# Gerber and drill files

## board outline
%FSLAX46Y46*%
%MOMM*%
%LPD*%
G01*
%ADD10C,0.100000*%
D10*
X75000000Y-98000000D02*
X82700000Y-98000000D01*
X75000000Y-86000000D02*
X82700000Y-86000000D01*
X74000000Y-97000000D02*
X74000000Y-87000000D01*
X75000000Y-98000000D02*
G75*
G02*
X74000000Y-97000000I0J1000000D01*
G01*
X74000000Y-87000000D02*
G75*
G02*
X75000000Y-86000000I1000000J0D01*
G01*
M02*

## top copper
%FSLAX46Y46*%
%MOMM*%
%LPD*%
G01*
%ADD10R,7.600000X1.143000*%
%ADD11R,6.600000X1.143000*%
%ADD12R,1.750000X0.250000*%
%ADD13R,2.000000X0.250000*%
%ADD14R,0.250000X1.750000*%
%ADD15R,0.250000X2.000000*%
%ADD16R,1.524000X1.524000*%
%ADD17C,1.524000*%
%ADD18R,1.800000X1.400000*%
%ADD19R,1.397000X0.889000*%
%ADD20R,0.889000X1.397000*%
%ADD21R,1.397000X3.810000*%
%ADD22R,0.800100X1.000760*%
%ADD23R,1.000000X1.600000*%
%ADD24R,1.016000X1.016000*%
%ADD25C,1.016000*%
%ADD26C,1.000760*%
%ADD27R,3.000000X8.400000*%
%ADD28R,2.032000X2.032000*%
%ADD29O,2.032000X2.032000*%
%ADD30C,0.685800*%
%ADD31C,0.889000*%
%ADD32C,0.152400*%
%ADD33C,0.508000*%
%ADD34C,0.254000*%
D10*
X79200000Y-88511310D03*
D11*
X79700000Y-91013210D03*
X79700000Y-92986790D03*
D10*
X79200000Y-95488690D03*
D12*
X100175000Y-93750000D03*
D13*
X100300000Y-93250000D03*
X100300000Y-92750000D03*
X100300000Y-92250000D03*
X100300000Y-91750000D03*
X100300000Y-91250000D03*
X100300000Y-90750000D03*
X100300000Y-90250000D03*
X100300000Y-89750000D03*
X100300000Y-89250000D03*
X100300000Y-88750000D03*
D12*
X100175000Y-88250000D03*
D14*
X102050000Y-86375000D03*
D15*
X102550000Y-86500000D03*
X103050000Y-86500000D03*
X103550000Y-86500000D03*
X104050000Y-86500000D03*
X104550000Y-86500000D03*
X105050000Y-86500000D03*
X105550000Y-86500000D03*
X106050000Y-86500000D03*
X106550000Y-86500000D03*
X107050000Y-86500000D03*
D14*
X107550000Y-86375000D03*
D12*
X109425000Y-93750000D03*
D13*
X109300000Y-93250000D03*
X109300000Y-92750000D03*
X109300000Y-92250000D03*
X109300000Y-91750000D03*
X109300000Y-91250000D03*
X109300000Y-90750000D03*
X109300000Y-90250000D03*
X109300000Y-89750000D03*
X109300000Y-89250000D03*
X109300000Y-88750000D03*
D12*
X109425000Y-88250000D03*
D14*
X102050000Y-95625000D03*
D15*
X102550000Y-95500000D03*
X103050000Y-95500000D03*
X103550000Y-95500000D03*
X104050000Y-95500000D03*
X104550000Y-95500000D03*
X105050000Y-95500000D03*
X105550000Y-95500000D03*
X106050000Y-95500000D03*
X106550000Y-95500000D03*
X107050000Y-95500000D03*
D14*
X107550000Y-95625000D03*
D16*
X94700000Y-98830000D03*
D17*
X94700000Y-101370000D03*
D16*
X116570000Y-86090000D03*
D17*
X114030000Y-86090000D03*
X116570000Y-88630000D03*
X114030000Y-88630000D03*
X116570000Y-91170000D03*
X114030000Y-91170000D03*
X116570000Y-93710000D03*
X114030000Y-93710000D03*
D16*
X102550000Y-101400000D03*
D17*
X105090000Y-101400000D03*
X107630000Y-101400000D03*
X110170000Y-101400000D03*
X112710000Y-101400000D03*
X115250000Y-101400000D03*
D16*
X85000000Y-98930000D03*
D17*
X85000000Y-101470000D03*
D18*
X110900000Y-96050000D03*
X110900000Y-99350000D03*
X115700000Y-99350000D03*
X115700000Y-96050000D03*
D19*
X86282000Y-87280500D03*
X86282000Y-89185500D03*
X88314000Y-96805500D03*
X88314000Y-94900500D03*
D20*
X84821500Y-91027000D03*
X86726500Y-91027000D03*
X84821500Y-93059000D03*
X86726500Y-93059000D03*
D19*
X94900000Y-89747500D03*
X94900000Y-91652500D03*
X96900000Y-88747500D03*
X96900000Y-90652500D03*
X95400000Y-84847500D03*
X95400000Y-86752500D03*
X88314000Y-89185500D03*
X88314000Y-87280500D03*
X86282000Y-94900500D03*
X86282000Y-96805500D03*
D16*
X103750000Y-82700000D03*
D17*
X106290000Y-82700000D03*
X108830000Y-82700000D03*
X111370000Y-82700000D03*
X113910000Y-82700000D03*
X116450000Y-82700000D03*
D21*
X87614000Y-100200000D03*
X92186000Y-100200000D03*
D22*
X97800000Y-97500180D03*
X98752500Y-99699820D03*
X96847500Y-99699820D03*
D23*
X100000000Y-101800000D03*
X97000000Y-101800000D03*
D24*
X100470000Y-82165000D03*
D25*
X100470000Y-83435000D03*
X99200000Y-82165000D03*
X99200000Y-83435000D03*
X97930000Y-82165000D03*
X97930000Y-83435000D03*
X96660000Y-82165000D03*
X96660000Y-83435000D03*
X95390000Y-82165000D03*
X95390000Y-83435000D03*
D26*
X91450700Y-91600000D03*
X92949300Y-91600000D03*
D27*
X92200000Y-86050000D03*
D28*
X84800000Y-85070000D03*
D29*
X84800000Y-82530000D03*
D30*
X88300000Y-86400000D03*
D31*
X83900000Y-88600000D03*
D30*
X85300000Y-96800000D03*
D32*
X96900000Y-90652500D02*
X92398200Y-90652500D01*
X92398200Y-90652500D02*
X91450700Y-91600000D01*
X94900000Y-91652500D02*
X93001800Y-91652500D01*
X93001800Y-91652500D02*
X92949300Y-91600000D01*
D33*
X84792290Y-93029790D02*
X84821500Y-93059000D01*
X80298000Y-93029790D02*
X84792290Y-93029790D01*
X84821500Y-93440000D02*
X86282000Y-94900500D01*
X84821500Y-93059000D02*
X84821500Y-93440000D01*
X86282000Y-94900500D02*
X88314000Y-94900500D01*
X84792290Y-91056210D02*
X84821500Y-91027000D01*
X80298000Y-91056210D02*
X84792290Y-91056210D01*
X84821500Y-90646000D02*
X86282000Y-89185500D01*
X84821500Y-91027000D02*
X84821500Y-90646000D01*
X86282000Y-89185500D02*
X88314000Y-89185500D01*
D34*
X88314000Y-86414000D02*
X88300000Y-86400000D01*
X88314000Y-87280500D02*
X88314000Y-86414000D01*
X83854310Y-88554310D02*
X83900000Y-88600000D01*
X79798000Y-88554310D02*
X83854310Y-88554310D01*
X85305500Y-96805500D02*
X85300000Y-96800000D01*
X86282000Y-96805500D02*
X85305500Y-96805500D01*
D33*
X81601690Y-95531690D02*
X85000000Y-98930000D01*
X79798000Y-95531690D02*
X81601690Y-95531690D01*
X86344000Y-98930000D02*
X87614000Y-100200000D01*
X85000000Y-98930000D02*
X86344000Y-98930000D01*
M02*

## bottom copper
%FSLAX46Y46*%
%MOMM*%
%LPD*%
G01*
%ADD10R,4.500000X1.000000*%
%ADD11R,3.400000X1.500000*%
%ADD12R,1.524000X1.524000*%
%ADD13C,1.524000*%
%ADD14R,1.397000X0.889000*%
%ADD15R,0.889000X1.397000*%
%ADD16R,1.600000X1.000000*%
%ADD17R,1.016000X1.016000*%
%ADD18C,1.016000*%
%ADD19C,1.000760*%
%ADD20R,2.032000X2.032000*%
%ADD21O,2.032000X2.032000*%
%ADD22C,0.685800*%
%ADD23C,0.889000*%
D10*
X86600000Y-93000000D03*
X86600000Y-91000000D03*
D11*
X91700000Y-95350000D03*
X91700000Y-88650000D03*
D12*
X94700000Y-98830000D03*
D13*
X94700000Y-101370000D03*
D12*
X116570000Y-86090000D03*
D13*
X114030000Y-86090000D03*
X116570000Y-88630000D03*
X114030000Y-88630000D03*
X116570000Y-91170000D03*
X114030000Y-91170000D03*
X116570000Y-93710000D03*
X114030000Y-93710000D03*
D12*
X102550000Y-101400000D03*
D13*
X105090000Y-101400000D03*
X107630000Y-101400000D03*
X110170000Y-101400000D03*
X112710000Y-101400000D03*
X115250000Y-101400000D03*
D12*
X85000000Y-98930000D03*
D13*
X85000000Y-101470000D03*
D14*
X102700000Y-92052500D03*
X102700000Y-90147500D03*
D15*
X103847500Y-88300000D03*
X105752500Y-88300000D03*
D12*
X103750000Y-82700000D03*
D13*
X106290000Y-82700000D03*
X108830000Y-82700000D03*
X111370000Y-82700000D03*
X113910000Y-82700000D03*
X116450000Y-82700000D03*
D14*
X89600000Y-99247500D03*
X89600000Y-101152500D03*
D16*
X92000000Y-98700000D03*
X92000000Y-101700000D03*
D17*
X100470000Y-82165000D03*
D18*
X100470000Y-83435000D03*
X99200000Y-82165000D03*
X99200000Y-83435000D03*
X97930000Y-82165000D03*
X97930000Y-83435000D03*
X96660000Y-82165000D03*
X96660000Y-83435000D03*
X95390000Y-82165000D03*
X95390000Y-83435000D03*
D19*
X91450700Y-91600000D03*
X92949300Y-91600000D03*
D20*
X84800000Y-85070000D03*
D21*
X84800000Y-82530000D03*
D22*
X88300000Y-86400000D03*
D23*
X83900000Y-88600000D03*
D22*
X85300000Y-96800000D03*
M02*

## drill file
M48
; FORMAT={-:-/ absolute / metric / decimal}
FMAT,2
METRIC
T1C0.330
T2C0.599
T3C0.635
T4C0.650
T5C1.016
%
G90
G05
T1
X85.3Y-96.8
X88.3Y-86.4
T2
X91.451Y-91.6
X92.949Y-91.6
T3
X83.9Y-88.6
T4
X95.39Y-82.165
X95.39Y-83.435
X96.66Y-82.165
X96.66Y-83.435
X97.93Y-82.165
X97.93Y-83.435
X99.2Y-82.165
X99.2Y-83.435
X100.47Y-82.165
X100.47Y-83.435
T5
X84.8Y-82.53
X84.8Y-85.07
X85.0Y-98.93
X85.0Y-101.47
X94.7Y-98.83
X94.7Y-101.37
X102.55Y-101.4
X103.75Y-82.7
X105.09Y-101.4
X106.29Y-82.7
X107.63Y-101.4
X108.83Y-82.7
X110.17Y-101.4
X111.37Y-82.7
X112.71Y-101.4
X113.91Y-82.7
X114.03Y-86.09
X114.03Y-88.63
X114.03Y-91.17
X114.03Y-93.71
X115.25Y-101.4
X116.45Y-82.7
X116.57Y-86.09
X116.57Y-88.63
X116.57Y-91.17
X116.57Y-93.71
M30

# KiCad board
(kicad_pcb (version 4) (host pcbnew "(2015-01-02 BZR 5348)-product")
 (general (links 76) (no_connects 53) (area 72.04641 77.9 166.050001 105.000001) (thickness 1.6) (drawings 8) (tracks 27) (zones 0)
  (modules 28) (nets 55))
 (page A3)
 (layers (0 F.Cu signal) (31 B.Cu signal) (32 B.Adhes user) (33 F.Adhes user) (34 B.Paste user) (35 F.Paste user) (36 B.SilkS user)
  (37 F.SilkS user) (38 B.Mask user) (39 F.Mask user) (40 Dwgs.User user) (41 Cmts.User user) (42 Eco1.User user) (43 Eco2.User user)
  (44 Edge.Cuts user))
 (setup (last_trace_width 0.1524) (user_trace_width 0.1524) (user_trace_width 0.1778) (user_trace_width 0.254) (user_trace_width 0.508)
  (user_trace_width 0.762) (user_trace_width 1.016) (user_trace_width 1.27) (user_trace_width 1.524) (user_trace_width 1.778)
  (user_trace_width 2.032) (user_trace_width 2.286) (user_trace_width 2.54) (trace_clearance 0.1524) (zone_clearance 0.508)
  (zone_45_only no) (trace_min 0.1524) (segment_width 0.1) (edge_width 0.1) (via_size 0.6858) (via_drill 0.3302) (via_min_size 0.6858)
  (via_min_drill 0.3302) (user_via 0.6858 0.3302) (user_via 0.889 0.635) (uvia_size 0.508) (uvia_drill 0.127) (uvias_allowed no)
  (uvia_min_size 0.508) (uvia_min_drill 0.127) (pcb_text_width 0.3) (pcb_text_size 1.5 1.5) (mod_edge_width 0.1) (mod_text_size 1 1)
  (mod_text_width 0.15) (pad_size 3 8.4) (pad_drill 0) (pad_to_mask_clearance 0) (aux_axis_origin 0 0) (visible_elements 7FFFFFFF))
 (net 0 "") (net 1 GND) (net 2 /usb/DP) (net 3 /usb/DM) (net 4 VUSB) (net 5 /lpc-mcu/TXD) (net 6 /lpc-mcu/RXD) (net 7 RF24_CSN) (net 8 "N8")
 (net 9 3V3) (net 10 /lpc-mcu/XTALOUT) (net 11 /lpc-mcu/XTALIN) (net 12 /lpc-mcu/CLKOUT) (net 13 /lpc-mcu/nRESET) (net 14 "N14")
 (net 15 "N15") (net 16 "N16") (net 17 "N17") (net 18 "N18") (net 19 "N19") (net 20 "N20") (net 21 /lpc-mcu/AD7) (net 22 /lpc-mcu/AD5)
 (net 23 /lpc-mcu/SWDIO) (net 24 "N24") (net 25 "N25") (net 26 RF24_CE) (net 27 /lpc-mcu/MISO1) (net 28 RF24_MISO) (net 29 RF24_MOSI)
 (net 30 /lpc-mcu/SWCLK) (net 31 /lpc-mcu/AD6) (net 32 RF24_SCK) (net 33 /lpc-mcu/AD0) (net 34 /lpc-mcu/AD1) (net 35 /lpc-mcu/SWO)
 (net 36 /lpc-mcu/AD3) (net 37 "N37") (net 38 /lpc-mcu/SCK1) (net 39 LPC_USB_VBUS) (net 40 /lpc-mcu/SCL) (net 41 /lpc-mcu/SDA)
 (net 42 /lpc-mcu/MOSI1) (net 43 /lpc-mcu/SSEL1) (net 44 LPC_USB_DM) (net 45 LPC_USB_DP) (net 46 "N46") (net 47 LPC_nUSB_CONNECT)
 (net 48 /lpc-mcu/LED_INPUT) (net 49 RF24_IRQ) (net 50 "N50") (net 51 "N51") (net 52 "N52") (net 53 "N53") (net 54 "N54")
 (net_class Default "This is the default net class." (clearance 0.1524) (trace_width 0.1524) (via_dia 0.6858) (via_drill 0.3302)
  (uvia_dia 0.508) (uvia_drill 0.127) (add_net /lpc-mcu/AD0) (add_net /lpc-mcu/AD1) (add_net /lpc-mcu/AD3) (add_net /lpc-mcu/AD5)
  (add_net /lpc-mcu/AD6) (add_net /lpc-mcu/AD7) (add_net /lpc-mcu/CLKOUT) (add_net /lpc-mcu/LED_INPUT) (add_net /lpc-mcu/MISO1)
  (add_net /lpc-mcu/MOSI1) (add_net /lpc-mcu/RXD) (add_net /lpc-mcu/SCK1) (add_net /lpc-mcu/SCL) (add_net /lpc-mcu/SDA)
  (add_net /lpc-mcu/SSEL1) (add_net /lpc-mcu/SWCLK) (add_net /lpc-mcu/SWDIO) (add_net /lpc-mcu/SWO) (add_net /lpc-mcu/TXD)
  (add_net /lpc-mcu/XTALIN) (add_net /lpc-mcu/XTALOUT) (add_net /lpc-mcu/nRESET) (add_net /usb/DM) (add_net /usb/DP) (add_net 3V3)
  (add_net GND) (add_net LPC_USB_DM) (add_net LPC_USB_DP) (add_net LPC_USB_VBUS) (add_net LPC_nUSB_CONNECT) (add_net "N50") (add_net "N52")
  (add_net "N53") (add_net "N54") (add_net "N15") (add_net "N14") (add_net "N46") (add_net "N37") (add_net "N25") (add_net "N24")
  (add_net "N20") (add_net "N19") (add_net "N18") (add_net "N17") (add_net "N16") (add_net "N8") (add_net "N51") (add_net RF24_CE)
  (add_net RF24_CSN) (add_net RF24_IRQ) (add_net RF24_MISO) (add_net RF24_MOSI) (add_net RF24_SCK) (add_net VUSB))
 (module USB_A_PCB (layer F.Cu) (at 74 92 270)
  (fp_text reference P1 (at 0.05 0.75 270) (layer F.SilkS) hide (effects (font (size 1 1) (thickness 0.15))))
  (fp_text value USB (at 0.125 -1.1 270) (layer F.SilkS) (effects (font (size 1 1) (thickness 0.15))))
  (pad 4 smd rect (at -3.48869 -5.2 270) (size 1.143 7.6) (layers F.Cu F.Paste F.Mask) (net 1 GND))
  (pad 3 smd rect (at -0.98679 -5.7 270) (size 1.143 6.6) (layers F.Cu F.Paste F.Mask) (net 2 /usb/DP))
  (pad 2 smd rect (at 0.98679 -5.7 270) (size 1.143 6.6) (layers F.Cu F.Paste F.Mask) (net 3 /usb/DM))
  (pad 1 smd rect (at 3.48869 -5.2 270) (size 1.143 7.6) (layers F.Cu F.Paste F.Mask) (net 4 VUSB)))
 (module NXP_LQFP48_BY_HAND (layer F.Cu) (at 104.8 91) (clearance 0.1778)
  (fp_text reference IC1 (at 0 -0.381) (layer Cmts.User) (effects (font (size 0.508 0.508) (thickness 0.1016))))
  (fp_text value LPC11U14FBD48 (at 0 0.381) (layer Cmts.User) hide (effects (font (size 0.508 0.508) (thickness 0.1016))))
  (pad 12 smd rect (at -4.625 2.75) (size 1.75 0.25) (layers F.Cu F.Paste F.Mask) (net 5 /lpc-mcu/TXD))
  (pad 11 smd rect (at -4.5 2.25) (size 2 0.25) (layers F.Cu F.Paste F.Mask) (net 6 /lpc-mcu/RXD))
  (pad 10 smd rect (at -4.5 1.75) (size 2 0.25) (layers F.Cu F.Paste F.Mask) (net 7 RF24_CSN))
  (pad 9 smd rect (at -4.5 1.25) (size 2 0.25) (layers F.Cu F.Paste F.Mask) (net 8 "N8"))
  (pad 8 smd rect (at -4.5 0.75) (size 2 0.25) (layers F.Cu F.Paste F.Mask) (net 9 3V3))
  (pad 7 smd rect (at -4.5 0.25) (size 2 0.25) (layers F.Cu F.Paste F.Mask) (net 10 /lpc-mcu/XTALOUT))
  (pad 6 smd rect (at -4.5 -0.25) (size 2 0.25) (layers F.Cu F.Paste F.Mask) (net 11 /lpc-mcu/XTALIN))
  (pad 5 smd rect (at -4.5 -0.75) (size 2 0.25) (layers F.Cu F.Paste F.Mask) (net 1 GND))
  (pad 4 smd rect (at -4.5 -1.25) (size 2 0.25) (layers F.Cu F.Paste F.Mask) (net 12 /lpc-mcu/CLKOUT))
  (pad 3 smd rect (at -4.5 -1.75) (size 2 0.25) (layers F.Cu F.Paste F.Mask) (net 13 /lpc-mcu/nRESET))
  (pad 2 smd rect (at -4.5 -2.25) (size 2 0.25) (layers F.Cu F.Paste F.Mask) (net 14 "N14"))
  (pad 1 smd rect (at -4.625 -2.75) (size 1.75 0.25) (layers F.Cu F.Paste F.Mask) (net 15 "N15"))
  (pad 48 smd rect (at -2.75 -4.625) (size 0.25 1.75) (layers F.Cu F.Paste F.Mask) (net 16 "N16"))
  (pad 47 smd rect (at -2.25 -4.5) (size 0.25 2) (layers F.Cu F.Paste F.Mask) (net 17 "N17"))
  (pad 46 smd rect (at -1.75 -4.5) (size 0.25 2) (layers F.Cu F.Paste F.Mask) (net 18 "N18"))
  (pad 45 smd rect (at -1.25 -4.5) (size 0.25 2) (layers F.Cu F.Paste F.Mask) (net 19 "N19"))
  (pad 44 smd rect (at -0.75 -4.5) (size 0.25 2) (layers F.Cu F.Paste F.Mask) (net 9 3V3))
  (pad 43 smd rect (at -0.25 -4.5) (size 0.25 2) (layers F.Cu F.Paste F.Mask) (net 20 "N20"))
  (pad 42 smd rect (at 0.25 -4.5) (size 0.25 2) (layers F.Cu F.Paste F.Mask) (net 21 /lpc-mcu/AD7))
  (pad 41 smd rect (at 0.75 -4.5) (size 0.25 2) (layers F.Cu F.Paste F.Mask) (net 1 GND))
  (pad 40 smd rect (at 1.25 -4.5) (size 0.25 2) (layers F.Cu F.Paste F.Mask) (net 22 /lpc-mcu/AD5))
  (pad 39 smd rect (at 1.75 -4.5) (size 0.25 2) (layers F.Cu F.Paste F.Mask) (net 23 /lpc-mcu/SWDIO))
  (pad 38 smd rect (at 2.25 -4.5) (size 0.25 2) (layers F.Cu F.Paste F.Mask) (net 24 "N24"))
  (pad 37 smd rect (at 2.75 -4.625) (size 0.25 1.75) (layers F.Cu F.Paste F.Mask) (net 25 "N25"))
  (pad 25 smd rect (at 4.625 2.75) (size 1.75 0.25) (layers F.Cu F.Paste F.Mask) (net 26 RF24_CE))
  (pad 26 smd rect (at 4.5 2.25) (size 2 0.25) (layers F.Cu F.Paste F.Mask) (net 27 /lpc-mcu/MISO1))
  (pad 27 smd rect (at 4.5 1.75) (size 2 0.25) (layers F.Cu F.Paste F.Mask) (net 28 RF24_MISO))
  (pad 28 smd rect (at 4.5 1.25) (size 2 0.25) (layers F.Cu F.Paste F.Mask) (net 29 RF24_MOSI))
  (pad 29 smd rect (at 4.5 0.75) (size 2 0.25) (layers F.Cu F.Paste F.Mask) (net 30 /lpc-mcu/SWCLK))
  (pad 30 smd rect (at 4.5 0.25) (size 2 0.25) (layers F.Cu F.Paste F.Mask) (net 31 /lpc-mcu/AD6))
  (pad 31 smd rect (at 4.5 -0.25) (size 2 0.25) (layers F.Cu F.Paste F.Mask) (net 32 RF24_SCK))
  (pad 32 smd rect (at 4.5 -0.75) (size 2 0.25) (layers F.Cu F.Paste F.Mask) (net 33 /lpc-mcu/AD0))
  (pad 33 smd rect (at 4.5 -1.25) (size 2 0.25) (layers F.Cu F.Paste F.Mask) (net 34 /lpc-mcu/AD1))
  (pad 34 smd rect (at 4.5 -1.75) (size 2 0.25) (layers F.Cu F.Paste F.Mask) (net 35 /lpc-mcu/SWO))
  (pad 35 smd rect (at 4.5 -2.25) (size 2 0.25) (layers F.Cu F.Paste F.Mask) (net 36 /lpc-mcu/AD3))
  (pad 36 smd rect (at 4.625 -2.75) (size 1.75 0.25) (layers F.Cu F.Paste F.Mask) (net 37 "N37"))
  (pad 13 smd rect (at -2.75 4.625) (size 0.25 1.75) (layers F.Cu F.Paste F.Mask) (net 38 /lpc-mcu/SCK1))
  (pad 14 smd rect (at -2.25 4.5) (size 0.25 2) (layers F.Cu F.Paste F.Mask) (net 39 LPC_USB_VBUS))
  (pad 15 smd rect (at -1.75 4.5) (size 0.25 2) (layers F.Cu F.Paste F.Mask) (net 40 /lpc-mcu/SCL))
  (pad 16 smd rect (at -1.25 4.5) (size 0.25 2) (layers F.Cu F.Paste F.Mask) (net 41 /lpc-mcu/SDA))
  (pad 17 smd rect (at -0.75 4.5) (size 0.25 2) (layers F.Cu F.Paste F.Mask) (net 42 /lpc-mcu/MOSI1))
  (pad 18 smd rect (at -0.25 4.5) (size 0.25 2) (layers F.Cu F.Paste F.Mask) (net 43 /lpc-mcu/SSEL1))
  (pad 19 smd rect (at 0.25 4.5) (size 0.25 2) (layers F.Cu F.Paste F.Mask) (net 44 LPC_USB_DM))
  (pad 20 smd rect (at 0.75 4.5) (size 0.25 2) (layers F.Cu F.Paste F.Mask) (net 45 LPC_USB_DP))
  (pad 21 smd rect (at 1.25 4.5) (size 0.25 2) (layers F.Cu F.Paste F.Mask) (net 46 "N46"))
  (pad 22 smd rect (at 1.75 4.5) (size 0.25 2) (layers F.Cu F.Paste F.Mask) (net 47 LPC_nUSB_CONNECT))
  (pad 23 smd rect (at 2.25 4.5) (size 0.25 2) (layers F.Cu F.Paste F.Mask) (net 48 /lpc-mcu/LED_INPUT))
  (pad 24 smd rect (at 2.75 4.625) (size 0.25 1.75) (layers F.Cu F.Paste F.Mask) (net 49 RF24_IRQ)))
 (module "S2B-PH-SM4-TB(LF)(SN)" (layer B.Cu) (at 86.6 92 90)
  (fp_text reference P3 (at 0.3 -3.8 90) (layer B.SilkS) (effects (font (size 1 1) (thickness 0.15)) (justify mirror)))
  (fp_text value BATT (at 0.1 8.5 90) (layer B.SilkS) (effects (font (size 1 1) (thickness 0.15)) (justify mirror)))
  (pad 1 smd rect (at -1 0 90) (size 1 4.5) (layers B.Cu B.Paste B.Mask) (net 1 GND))
  (pad 2 smd rect (at 1 0 90) (size 1 4.5) (layers B.Cu B.Paste B.Mask) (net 4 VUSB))
  (pad NC smd rect (at -3.35 5.1 90) (size 1.5 3.4) (layers B.Cu B.Paste B.Mask))
  (pad NC smd rect (at 3.35 5.1 90) (size 1.5 3.4) (layers B.Cu B.Paste B.Mask)))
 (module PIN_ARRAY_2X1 (layer F.Cu) (at 94.7 100.1 270)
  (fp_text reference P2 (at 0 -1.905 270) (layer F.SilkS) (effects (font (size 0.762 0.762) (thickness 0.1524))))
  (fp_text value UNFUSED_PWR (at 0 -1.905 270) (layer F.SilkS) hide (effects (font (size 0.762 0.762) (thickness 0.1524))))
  (pad 1 thru_hole rect (at -1.27 0 270) (size 1.524 1.524) (drill 1.016) (layers *.Cu *.Mask F.SilkS) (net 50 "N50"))
  (pad 2 thru_hole circle (at 1.27 0 270) (size 1.524 1.524) (drill 1.016) (layers *.Cu *.Mask F.SilkS) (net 1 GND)))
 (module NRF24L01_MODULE (layer B.Cu) (at 115.3 89.9 270)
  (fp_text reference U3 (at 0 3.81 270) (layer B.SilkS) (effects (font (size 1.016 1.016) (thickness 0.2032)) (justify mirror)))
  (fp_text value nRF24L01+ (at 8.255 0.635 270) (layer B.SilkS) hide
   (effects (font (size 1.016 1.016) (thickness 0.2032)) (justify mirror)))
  (pad 1 thru_hole rect (at -3.81 -1.27 270) (size 1.524 1.524) (drill 1.016) (layers *.Cu *.Mask B.SilkS) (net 1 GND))
  (pad 2 thru_hole circle (at -3.81 1.27 270) (size 1.524 1.524) (drill 1.016) (layers *.Cu *.Mask B.SilkS) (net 9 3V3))
  (pad 3 thru_hole circle (at -1.27 -1.27 270) (size 1.524 1.524) (drill 1.016) (layers *.Cu *.Mask B.SilkS) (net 26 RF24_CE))
  (pad 4 thru_hole circle (at -1.27 1.27 270) (size 1.524 1.524) (drill 1.016) (layers *.Cu *.Mask B.SilkS) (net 7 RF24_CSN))
  (pad 5 thru_hole circle (at 1.27 -1.27 270) (size 1.524 1.524) (drill 1.016) (layers *.Cu *.Mask B.SilkS) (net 32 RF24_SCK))
  (pad 6 thru_hole circle (at 1.27 1.27 270) (size 1.524 1.524) (drill 1.016) (layers *.Cu *.Mask B.SilkS) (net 29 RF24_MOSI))
  (pad 7 thru_hole circle (at 3.81 -1.27 270) (size 1.524 1.524) (drill 1.016) (layers *.Cu *.Mask B.SilkS) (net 28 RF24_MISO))
  (pad 8 thru_hole circle (at 3.81 1.27 270) (size 1.524 1.524) (drill 1.016) (layers *.Cu *.Mask B.SilkS) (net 49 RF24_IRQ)))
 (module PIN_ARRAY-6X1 (layer F.Cu) (at 108.9 101.4)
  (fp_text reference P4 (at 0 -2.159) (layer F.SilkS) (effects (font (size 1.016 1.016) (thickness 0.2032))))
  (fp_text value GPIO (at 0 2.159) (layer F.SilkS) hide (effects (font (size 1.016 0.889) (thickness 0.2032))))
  (pad 1 thru_hole rect (at -6.35 0) (size 1.524 1.524) (drill 1.016) (layers *.Cu *.Mask F.SilkS) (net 1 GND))
  (pad 2 thru_hole circle (at -3.81 0) (size 1.524 1.524) (drill 1.016) (layers *.Cu *.Mask F.SilkS) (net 9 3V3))
  (pad 3 thru_hole circle (at -1.27 0) (size 1.524 1.524) (drill 1.016) (layers *.Cu *.Mask F.SilkS) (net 40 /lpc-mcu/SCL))
  (pad 4 thru_hole circle (at 1.27 0) (size 1.524 1.524) (drill 1.016) (layers *.Cu *.Mask F.SilkS) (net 41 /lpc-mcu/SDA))
  (pad 5 thru_hole circle (at 3.81 0) (size 1.524 1.524) (drill 1.016) (layers *.Cu *.Mask F.SilkS) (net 6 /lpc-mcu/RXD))
  (pad 6 thru_hole circle (at 6.35 0) (size 1.524 1.524) (drill 1.016) (layers *.Cu *.Mask F.SilkS) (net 5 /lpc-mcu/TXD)))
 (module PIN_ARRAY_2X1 (layer F.Cu) (at 85 100.2 270)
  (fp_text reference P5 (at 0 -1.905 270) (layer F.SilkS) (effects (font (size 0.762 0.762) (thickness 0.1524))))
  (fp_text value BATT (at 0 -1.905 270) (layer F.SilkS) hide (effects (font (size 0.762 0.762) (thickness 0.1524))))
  (pad 1 thru_hole rect (at -1.27 0 270) (size 1.524 1.524) (drill 1.016) (layers *.Cu *.Mask F.SilkS) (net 4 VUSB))
  (pad 2 thru_hole circle (at 1.27 0 270) (size 1.524 1.524) (drill 1.016) (layers *.Cu *.Mask F.SilkS) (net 1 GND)))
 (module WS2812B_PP (layer F.Cu) (at 113.3 97.7 90)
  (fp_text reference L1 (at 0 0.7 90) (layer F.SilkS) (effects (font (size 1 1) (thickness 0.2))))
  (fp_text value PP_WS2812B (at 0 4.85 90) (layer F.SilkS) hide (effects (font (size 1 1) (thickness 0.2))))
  (pad 3 smd rect (at 1.65 -2.4 90) (size 1.4 1.8) (layers F.Cu F.Paste F.Mask) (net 1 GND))
  (pad 4 smd rect (at -1.65 -2.4 90) (size 1.4 1.8) (layers F.Cu F.Paste F.Mask) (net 48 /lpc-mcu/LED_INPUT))
  (pad 1 smd rect (at -1.65 2.4 90) (size 1.4 1.8) (layers F.Cu F.Paste F.Mask) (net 9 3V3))
  (pad 2 smd rect (at 1.65 2.4 90) (size 1.4 1.8) (layers F.Cu F.Paste F.Mask) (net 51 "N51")))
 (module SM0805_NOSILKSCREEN (layer B.Cu) (at 102.7 91.1 90)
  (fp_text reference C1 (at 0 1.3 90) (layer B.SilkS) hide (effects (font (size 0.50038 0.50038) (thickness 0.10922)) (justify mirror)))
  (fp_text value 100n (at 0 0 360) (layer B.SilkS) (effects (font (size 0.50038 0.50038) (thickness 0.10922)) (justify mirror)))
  (pad 1 smd rect (at -0.9525 0 90) (size 0.889 1.397) (layers B.Cu B.Paste B.Mask) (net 9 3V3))
  (pad 2 smd rect (at 0.9525 0 90) (size 0.889 1.397) (layers B.Cu B.Paste B.Mask) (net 1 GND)))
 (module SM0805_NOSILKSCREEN (layer F.Cu) (at 86.282 88.233 270)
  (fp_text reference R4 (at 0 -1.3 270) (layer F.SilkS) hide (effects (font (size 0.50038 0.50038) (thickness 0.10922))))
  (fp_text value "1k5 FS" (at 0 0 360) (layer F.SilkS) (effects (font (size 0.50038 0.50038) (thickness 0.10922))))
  (pad 1 smd rect (at -0.9525 0 270) (size 0.889 1.397) (layers F.Cu F.Paste F.Mask) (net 9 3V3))
  (pad 2 smd rect (at 0.9525 0 270) (size 0.889 1.397) (layers F.Cu F.Paste F.Mask) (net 2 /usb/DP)))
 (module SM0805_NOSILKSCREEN (layer F.Cu) (at 88.314 95.853 90)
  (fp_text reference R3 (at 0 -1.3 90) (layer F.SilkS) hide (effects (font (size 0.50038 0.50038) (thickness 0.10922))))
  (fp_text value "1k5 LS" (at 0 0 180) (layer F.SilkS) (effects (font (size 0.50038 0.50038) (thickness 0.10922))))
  (pad 1 smd rect (at -0.9525 0 90) (size 0.889 1.397) (layers F.Cu F.Paste F.Mask) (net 9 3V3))
  (pad 2 smd rect (at 0.9525 0 90) (size 0.889 1.397) (layers F.Cu F.Paste F.Mask) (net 3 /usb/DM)))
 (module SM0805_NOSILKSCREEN (layer F.Cu) (at 85.774 91.027)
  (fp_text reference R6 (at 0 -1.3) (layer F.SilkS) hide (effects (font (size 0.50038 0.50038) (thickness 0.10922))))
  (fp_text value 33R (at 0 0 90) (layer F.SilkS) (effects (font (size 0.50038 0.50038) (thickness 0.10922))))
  (pad 1 smd rect (at -0.9525 0) (size 0.889 1.397) (layers F.Cu F.Paste F.Mask) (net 2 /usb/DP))
  (pad 2 smd rect (at 0.9525 0) (size 0.889 1.397) (layers F.Cu F.Paste F.Mask) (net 45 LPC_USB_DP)))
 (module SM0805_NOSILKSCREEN (layer F.Cu) (at 85.774 93.059)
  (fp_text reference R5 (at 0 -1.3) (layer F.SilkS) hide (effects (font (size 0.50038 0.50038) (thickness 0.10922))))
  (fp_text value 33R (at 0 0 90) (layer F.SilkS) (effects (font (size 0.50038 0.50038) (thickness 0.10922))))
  (pad 1 smd rect (at -0.9525 0) (size 0.889 1.397) (layers F.Cu F.Paste F.Mask) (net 3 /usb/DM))
  (pad 2 smd rect (at 0.9525 0) (size 0.889 1.397) (layers F.Cu F.Paste F.Mask) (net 44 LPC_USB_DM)))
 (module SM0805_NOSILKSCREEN (layer F.Cu) (at 94.9 90.7 270)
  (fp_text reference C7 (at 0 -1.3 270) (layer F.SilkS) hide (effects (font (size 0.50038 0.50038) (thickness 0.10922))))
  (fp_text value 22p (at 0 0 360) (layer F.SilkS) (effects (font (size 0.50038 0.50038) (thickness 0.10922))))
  (pad 1 smd rect (at -0.9525 0 270) (size 0.889 1.397) (layers F.Cu F.Paste F.Mask) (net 1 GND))
  (pad 2 smd rect (at 0.9525 0 270) (size 0.889 1.397) (layers F.Cu F.Paste F.Mask) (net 10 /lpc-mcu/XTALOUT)))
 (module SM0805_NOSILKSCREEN (layer F.Cu) (at 96.9 89.7 270)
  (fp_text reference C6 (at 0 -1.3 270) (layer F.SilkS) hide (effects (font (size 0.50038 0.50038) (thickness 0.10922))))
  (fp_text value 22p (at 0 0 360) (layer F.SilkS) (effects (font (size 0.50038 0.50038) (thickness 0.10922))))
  (pad 1 smd rect (at -0.9525 0 270) (size 0.889 1.397) (layers F.Cu F.Paste F.Mask) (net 1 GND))
  (pad 2 smd rect (at 0.9525 0 270) (size 0.889 1.397) (layers F.Cu F.Paste F.Mask) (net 11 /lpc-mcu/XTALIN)))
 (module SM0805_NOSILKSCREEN (layer F.Cu) (at 95.4 85.8 270)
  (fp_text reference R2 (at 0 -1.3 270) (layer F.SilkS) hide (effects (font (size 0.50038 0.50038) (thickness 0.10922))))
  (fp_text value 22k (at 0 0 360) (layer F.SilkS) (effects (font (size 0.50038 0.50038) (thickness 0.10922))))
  (pad 1 smd rect (at -0.9525 0 270) (size 0.889 1.397) (layers F.Cu F.Paste F.Mask) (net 13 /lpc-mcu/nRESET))
  (pad 2 smd rect (at 0.9525 0 270) (size 0.889 1.397) (layers F.Cu F.Paste F.Mask) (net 9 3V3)))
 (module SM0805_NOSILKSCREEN (layer B.Cu) (at 104.8 88.3)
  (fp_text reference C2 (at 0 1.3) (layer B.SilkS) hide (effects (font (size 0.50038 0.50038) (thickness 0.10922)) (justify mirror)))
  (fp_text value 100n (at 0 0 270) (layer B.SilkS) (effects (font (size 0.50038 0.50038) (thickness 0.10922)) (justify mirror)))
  (pad 1 smd rect (at -0.9525 0) (size 0.889 1.397) (layers B.Cu B.Paste B.Mask) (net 9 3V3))
  (pad 2 smd rect (at 0.9525 0) (size 0.889 1.397) (layers B.Cu B.Paste B.Mask) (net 1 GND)))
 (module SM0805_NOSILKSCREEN (layer F.Cu) (at 88.314 88.233 90)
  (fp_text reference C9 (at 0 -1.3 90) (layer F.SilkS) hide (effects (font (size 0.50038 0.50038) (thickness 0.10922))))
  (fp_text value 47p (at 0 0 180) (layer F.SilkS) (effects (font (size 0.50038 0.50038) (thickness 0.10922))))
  (pad 1 smd rect (at -0.9525 0 90) (size 0.889 1.397) (layers F.Cu F.Paste F.Mask) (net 2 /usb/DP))
  (pad 2 smd rect (at 0.9525 0 90) (size 0.889 1.397) (layers F.Cu F.Paste F.Mask) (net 1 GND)))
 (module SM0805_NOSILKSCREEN (layer F.Cu) (at 86.282 95.853 270)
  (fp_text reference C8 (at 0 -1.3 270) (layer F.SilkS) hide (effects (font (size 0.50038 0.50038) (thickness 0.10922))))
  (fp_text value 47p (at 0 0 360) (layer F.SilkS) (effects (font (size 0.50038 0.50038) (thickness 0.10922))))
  (pad 1 smd rect (at -0.9525 0 270) (size 0.889 1.397) (layers F.Cu F.Paste F.Mask) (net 3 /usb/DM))
  (pad 2 smd rect (at 0.9525 0 270) (size 0.889 1.397) (layers F.Cu F.Paste F.Mask) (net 1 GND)))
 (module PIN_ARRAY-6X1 (layer F.Cu) (at 110.1 82.7)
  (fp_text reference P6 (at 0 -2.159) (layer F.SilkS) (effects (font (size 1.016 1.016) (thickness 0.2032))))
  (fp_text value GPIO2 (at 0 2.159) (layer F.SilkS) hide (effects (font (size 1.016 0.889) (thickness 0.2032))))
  (pad 1 thru_hole rect (at -6.35 0) (size 1.524 1.524) (drill 1.016) (layers *.Cu *.Mask F.SilkS) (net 33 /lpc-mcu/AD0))
  (pad 2 thru_hole circle (at -3.81 0) (size 1.524 1.524) (drill 1.016) (layers *.Cu *.Mask F.SilkS) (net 34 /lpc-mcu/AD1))
  (pad 3 thru_hole circle (at -1.27 0) (size 1.524 1.524) (drill 1.016) (layers *.Cu *.Mask F.SilkS) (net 43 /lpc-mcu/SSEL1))
  (pad 4 thru_hole circle (at 1.27 0) (size 1.524 1.524) (drill 1.016) (layers *.Cu *.Mask F.SilkS) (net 27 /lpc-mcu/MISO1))
  (pad 5 thru_hole circle (at 3.81 0) (size 1.524 1.524) (drill 1.016) (layers *.Cu *.Mask F.SilkS) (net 42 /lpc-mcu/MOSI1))
  (pad 6 thru_hole circle (at 6.35 0) (size 1.524 1.524) (drill 1.016) (layers *.Cu *.Mask F.SilkS) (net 38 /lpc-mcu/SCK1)))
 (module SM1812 (layer F.Cu) (at 89.9 100.2)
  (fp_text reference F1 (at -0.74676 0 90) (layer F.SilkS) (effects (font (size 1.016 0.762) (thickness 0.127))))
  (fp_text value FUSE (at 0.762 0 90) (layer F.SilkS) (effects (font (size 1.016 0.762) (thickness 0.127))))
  (pad 1 smd rect (at -2.286 0) (size 1.397 3.81) (layers F.Cu F.Paste F.Mask) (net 4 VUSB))
  (pad 2 smd rect (at 2.286 0) (size 1.397 3.81) (layers F.Cu F.Paste F.Mask) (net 50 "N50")))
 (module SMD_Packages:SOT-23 (layer F.Cu) (at 97.8 98.6)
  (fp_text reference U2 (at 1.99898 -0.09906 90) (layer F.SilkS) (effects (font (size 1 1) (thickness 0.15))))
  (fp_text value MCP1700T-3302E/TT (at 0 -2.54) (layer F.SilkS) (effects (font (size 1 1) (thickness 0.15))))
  (pad 3 smd rect (at 0 -1.09982) (size 0.8001 1.00076) (layers F.Cu F.Paste F.Mask) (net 50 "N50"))
  (pad 2 smd rect (at 0.9525 1.09982) (size 0.8001 1.00076) (layers F.Cu F.Paste F.Mask) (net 9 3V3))
  (pad 1 smd rect (at -0.9525 1.09982) (size 0.8001 1.00076) (layers F.Cu F.Paste F.Mask) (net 1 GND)))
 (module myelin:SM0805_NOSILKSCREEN (layer B.Cu) (at 89.6 100.2 270)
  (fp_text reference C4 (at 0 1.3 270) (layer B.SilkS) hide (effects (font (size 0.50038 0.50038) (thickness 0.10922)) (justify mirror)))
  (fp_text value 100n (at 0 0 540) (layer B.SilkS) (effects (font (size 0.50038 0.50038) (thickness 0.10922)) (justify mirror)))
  (pad 1 smd rect (at -0.9525 0 270) (size 0.889 1.397) (layers B.Cu B.Paste B.Mask) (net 50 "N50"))
  (pad 2 smd rect (at 0.9525 0 270) (size 0.889 1.397) (layers B.Cu B.Paste B.Mask) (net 1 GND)))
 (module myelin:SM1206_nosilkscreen (layer B.Cu) (at 92 100.2 270)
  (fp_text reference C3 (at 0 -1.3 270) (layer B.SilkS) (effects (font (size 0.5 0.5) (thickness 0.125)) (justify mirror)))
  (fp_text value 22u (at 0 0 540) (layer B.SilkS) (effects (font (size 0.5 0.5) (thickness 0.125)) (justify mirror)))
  (pad 1 smd rect (at -1.5 0 270) (size 1 1.6) (layers B.Cu B.Paste B.Mask) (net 50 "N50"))
  (pad 2 smd rect (at 1.5 0 270) (size 1 1.6) (layers B.Cu B.Paste B.Mask) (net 1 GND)))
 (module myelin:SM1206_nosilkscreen (layer F.Cu) (at 98.5 101.8 180)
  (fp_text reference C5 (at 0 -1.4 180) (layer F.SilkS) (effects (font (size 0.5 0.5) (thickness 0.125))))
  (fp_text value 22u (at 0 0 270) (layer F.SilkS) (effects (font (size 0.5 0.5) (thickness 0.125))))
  (pad 1 smd rect (at -1.5 0 180) (size 1 1.6) (layers F.Cu F.Paste F.Mask) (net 9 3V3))
  (pad 2 smd rect (at 1.5 0 180) (size 1 1.6) (layers F.Cu F.Paste F.Mask) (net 1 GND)))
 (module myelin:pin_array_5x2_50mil (layer F.Cu) (at 99.2 82.8 180)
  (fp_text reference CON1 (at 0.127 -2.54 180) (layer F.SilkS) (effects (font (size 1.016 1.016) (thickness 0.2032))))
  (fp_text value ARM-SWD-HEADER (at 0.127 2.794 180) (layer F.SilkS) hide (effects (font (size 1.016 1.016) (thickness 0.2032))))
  (pad 1 thru_hole rect (at -1.27 0.635 180) (size 1.016 1.016) (drill 0.65) (layers *.Cu *.Mask F.SilkS) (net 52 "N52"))
  (pad 2 thru_hole circle (at -1.27 -0.635 180) (size 1.016 1.016) (drill 0.65) (layers *.Cu *.Mask F.SilkS) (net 23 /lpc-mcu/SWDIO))
  (pad 3 thru_hole circle (at 0 0.635 180) (size 1.016 1.016) (drill 0.65) (layers *.Cu *.Mask F.SilkS) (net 1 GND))
  (pad 4 thru_hole circle (at 0 -0.635 180) (size 1.016 1.016) (drill 0.65) (layers *.Cu *.Mask F.SilkS) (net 30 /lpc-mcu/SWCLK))
  (pad 5 thru_hole circle (at 1.27 0.635 180) (size 1.016 1.016) (drill 0.65) (layers *.Cu *.Mask F.SilkS) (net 1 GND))
  (pad 6 thru_hole circle (at 1.27 -0.635 180) (size 1.016 1.016) (drill 0.65) (layers *.Cu *.Mask F.SilkS) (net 35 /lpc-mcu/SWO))
  (pad 7 thru_hole circle (at 2.54 0.635 180) (size 1.016 1.016) (drill 0.65) (layers *.Cu *.Mask F.SilkS) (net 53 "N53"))
  (pad 8 thru_hole circle (at 2.54 -0.635 180) (size 1.016 1.016) (drill 0.65) (layers *.Cu *.Mask F.SilkS) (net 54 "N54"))
  (pad 9 thru_hole circle (at 3.81 0.635 180) (size 1.016 1.016) (drill 0.65) (layers *.Cu *.Mask F.SilkS) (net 1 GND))
  (pad 10 thru_hole circle (at 3.81 -0.635 180) (size 1.016 1.016) (drill 0.65) (layers *.Cu *.Mask F.SilkS) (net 13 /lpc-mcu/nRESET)))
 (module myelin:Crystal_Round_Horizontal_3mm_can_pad (layer F.Cu) (at 92.2 91.6)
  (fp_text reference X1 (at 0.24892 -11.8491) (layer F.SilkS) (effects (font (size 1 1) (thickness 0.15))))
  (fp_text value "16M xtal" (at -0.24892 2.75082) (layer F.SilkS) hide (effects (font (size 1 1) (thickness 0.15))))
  (pad 1 thru_hole circle (at -0.7493 0) (size 1.00076 1.00076) (drill 0.59944) (layers *.Cu *.Mask F.SilkS) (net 11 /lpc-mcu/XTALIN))
  (pad 2 thru_hole circle (at 0.7493 0) (size 1.00076 1.00076) (drill 0.59944) (layers *.Cu *.Mask F.SilkS) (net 10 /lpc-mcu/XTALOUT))
  (pad 3 smd rect (at 0 -5.55) (size 3 8.4) (layers F.Cu F.Paste F.Mask) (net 1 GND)))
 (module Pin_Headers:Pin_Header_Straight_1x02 (layer F.Cu) (at 84.8 83.8 90)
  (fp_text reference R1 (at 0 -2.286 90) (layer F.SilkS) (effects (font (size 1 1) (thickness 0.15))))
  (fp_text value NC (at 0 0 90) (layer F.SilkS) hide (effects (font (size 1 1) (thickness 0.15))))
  (pad 1 thru_hole rect (at -1.27 0 90) (size 2.032 2.032) (drill 1.016) (layers *.Cu *.Mask F.SilkS) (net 9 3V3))
  (pad 2 thru_hole oval (at 1.27 0 90) (size 2.032 2.032) (drill 1.016) (layers *.Cu *.Mask F.SilkS) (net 52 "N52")))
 (gr_line (start 75 98) (end 82.7 98) (angle 90) (layer Edge.Cuts) (width 0.1))
 (gr_line (start 75 86) (end 82.7 86) (angle 90) (layer Edge.Cuts) (width 0.1))
 (gr_line (start 74 97) (end 74 87) (angle 90) (layer Edge.Cuts) (width 0.1))
 (gr_arc (start 75 97) (end 75 98) (angle 90) (layer Edge.Cuts) (width 0.1))
 (gr_arc (start 75 87) (end 74 87) (angle 90) (layer Edge.Cuts) (width 0.1))
 (segment (start 96.9 90.6525) (end 92.3982 90.6525) (width 0.1524) (layer F.Cu) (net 11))
 (segment (start 92.3982 90.6525) (end 91.4507 91.6) (width 0.1524) (layer F.Cu) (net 11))
 (segment (start 94.9 91.6525) (end 93.0018 91.6525) (width 0.1524) (layer F.Cu) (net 10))
 (segment (start 93.0018 91.6525) (end 92.9493 91.6) (width 0.1524) (layer F.Cu) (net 10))
 (segment (start 84.79229 93.02979) (end 84.8215 93.059) (width 0.508) (layer F.Cu) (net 3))
 (segment (start 80.298 93.02979) (end 84.79229 93.02979) (width 0.508) (layer F.Cu) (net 3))
 (segment (start 84.8215 93.44) (end 86.282 94.9005) (width 0.508) (layer F.Cu) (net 3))
 (segment (start 84.8215 93.059) (end 84.8215 93.44) (width 0.508) (layer F.Cu) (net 3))
 (segment (start 86.282 94.9005) (end 88.314 94.9005) (width 0.508) (layer F.Cu) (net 3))
 (segment (start 84.79229 91.05621) (end 84.8215 91.027) (width 0.508) (layer F.Cu) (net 2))
 (segment (start 80.298 91.05621) (end 84.79229 91.05621) (width 0.508) (layer F.Cu) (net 2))
 (segment (start 84.8215 90.646) (end 86.282 89.1855) (width 0.508) (layer F.Cu) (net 2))
 (segment (start 84.8215 91.027) (end 84.8215 90.646) (width 0.508) (layer F.Cu) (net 2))
 (segment (start 86.282 89.1855) (end 88.314 89.1855) (width 0.508) (layer F.Cu) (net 2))
 (segment (start 88.314 86.414) (end 88.3 86.4) (width 0.254) (layer F.Cu) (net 1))
 (via (at 88.3 86.4) (size 0.6858) (drill 0.3302) (layers F.Cu B.Cu) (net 1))
 (segment (start 88.314 87.2805) (end 88.314 86.414) (width 0.254) (layer F.Cu) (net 1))
 (segment (start 83.85431 88.55431) (end 83.9 88.6) (width 0.254) (layer F.Cu) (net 1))
 (via (at 83.9 88.6) (size 0.889) (drill 0.635) (layers F.Cu B.Cu) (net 1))
 (segment (start 79.798 88.55431) (end 83.85431 88.55431) (width 0.254) (layer F.Cu) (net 1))
 (segment (start 85.3055 96.8055) (end 85.3 96.8) (width 0.254) (layer F.Cu) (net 1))
 (via (at 85.3 96.8) (size 0.6858) (drill 0.3302) (layers F.Cu B.Cu) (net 1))
 (segment (start 86.282 96.8055) (end 85.3055 96.8055) (width 0.254) (layer F.Cu) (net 1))
 (segment (start 81.60169 95.53169) (end 85 98.93) (width 0.508) (layer F.Cu) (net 4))
 (segment (start 79.798 95.53169) (end 81.60169 95.53169) (width 0.508) (layer F.Cu) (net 4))
 (segment (start 86.344 98.93) (end 87.614 100.2) (width 0.508) (layer F.Cu) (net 4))
 (segment (start 85 98.93) (end 86.344 98.93) (width 0.508) (layer F.Cu) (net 4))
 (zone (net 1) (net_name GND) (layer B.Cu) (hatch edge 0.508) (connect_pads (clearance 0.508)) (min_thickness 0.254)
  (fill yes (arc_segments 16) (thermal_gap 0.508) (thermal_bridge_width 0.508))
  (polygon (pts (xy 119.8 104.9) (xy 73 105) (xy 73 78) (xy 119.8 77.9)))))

